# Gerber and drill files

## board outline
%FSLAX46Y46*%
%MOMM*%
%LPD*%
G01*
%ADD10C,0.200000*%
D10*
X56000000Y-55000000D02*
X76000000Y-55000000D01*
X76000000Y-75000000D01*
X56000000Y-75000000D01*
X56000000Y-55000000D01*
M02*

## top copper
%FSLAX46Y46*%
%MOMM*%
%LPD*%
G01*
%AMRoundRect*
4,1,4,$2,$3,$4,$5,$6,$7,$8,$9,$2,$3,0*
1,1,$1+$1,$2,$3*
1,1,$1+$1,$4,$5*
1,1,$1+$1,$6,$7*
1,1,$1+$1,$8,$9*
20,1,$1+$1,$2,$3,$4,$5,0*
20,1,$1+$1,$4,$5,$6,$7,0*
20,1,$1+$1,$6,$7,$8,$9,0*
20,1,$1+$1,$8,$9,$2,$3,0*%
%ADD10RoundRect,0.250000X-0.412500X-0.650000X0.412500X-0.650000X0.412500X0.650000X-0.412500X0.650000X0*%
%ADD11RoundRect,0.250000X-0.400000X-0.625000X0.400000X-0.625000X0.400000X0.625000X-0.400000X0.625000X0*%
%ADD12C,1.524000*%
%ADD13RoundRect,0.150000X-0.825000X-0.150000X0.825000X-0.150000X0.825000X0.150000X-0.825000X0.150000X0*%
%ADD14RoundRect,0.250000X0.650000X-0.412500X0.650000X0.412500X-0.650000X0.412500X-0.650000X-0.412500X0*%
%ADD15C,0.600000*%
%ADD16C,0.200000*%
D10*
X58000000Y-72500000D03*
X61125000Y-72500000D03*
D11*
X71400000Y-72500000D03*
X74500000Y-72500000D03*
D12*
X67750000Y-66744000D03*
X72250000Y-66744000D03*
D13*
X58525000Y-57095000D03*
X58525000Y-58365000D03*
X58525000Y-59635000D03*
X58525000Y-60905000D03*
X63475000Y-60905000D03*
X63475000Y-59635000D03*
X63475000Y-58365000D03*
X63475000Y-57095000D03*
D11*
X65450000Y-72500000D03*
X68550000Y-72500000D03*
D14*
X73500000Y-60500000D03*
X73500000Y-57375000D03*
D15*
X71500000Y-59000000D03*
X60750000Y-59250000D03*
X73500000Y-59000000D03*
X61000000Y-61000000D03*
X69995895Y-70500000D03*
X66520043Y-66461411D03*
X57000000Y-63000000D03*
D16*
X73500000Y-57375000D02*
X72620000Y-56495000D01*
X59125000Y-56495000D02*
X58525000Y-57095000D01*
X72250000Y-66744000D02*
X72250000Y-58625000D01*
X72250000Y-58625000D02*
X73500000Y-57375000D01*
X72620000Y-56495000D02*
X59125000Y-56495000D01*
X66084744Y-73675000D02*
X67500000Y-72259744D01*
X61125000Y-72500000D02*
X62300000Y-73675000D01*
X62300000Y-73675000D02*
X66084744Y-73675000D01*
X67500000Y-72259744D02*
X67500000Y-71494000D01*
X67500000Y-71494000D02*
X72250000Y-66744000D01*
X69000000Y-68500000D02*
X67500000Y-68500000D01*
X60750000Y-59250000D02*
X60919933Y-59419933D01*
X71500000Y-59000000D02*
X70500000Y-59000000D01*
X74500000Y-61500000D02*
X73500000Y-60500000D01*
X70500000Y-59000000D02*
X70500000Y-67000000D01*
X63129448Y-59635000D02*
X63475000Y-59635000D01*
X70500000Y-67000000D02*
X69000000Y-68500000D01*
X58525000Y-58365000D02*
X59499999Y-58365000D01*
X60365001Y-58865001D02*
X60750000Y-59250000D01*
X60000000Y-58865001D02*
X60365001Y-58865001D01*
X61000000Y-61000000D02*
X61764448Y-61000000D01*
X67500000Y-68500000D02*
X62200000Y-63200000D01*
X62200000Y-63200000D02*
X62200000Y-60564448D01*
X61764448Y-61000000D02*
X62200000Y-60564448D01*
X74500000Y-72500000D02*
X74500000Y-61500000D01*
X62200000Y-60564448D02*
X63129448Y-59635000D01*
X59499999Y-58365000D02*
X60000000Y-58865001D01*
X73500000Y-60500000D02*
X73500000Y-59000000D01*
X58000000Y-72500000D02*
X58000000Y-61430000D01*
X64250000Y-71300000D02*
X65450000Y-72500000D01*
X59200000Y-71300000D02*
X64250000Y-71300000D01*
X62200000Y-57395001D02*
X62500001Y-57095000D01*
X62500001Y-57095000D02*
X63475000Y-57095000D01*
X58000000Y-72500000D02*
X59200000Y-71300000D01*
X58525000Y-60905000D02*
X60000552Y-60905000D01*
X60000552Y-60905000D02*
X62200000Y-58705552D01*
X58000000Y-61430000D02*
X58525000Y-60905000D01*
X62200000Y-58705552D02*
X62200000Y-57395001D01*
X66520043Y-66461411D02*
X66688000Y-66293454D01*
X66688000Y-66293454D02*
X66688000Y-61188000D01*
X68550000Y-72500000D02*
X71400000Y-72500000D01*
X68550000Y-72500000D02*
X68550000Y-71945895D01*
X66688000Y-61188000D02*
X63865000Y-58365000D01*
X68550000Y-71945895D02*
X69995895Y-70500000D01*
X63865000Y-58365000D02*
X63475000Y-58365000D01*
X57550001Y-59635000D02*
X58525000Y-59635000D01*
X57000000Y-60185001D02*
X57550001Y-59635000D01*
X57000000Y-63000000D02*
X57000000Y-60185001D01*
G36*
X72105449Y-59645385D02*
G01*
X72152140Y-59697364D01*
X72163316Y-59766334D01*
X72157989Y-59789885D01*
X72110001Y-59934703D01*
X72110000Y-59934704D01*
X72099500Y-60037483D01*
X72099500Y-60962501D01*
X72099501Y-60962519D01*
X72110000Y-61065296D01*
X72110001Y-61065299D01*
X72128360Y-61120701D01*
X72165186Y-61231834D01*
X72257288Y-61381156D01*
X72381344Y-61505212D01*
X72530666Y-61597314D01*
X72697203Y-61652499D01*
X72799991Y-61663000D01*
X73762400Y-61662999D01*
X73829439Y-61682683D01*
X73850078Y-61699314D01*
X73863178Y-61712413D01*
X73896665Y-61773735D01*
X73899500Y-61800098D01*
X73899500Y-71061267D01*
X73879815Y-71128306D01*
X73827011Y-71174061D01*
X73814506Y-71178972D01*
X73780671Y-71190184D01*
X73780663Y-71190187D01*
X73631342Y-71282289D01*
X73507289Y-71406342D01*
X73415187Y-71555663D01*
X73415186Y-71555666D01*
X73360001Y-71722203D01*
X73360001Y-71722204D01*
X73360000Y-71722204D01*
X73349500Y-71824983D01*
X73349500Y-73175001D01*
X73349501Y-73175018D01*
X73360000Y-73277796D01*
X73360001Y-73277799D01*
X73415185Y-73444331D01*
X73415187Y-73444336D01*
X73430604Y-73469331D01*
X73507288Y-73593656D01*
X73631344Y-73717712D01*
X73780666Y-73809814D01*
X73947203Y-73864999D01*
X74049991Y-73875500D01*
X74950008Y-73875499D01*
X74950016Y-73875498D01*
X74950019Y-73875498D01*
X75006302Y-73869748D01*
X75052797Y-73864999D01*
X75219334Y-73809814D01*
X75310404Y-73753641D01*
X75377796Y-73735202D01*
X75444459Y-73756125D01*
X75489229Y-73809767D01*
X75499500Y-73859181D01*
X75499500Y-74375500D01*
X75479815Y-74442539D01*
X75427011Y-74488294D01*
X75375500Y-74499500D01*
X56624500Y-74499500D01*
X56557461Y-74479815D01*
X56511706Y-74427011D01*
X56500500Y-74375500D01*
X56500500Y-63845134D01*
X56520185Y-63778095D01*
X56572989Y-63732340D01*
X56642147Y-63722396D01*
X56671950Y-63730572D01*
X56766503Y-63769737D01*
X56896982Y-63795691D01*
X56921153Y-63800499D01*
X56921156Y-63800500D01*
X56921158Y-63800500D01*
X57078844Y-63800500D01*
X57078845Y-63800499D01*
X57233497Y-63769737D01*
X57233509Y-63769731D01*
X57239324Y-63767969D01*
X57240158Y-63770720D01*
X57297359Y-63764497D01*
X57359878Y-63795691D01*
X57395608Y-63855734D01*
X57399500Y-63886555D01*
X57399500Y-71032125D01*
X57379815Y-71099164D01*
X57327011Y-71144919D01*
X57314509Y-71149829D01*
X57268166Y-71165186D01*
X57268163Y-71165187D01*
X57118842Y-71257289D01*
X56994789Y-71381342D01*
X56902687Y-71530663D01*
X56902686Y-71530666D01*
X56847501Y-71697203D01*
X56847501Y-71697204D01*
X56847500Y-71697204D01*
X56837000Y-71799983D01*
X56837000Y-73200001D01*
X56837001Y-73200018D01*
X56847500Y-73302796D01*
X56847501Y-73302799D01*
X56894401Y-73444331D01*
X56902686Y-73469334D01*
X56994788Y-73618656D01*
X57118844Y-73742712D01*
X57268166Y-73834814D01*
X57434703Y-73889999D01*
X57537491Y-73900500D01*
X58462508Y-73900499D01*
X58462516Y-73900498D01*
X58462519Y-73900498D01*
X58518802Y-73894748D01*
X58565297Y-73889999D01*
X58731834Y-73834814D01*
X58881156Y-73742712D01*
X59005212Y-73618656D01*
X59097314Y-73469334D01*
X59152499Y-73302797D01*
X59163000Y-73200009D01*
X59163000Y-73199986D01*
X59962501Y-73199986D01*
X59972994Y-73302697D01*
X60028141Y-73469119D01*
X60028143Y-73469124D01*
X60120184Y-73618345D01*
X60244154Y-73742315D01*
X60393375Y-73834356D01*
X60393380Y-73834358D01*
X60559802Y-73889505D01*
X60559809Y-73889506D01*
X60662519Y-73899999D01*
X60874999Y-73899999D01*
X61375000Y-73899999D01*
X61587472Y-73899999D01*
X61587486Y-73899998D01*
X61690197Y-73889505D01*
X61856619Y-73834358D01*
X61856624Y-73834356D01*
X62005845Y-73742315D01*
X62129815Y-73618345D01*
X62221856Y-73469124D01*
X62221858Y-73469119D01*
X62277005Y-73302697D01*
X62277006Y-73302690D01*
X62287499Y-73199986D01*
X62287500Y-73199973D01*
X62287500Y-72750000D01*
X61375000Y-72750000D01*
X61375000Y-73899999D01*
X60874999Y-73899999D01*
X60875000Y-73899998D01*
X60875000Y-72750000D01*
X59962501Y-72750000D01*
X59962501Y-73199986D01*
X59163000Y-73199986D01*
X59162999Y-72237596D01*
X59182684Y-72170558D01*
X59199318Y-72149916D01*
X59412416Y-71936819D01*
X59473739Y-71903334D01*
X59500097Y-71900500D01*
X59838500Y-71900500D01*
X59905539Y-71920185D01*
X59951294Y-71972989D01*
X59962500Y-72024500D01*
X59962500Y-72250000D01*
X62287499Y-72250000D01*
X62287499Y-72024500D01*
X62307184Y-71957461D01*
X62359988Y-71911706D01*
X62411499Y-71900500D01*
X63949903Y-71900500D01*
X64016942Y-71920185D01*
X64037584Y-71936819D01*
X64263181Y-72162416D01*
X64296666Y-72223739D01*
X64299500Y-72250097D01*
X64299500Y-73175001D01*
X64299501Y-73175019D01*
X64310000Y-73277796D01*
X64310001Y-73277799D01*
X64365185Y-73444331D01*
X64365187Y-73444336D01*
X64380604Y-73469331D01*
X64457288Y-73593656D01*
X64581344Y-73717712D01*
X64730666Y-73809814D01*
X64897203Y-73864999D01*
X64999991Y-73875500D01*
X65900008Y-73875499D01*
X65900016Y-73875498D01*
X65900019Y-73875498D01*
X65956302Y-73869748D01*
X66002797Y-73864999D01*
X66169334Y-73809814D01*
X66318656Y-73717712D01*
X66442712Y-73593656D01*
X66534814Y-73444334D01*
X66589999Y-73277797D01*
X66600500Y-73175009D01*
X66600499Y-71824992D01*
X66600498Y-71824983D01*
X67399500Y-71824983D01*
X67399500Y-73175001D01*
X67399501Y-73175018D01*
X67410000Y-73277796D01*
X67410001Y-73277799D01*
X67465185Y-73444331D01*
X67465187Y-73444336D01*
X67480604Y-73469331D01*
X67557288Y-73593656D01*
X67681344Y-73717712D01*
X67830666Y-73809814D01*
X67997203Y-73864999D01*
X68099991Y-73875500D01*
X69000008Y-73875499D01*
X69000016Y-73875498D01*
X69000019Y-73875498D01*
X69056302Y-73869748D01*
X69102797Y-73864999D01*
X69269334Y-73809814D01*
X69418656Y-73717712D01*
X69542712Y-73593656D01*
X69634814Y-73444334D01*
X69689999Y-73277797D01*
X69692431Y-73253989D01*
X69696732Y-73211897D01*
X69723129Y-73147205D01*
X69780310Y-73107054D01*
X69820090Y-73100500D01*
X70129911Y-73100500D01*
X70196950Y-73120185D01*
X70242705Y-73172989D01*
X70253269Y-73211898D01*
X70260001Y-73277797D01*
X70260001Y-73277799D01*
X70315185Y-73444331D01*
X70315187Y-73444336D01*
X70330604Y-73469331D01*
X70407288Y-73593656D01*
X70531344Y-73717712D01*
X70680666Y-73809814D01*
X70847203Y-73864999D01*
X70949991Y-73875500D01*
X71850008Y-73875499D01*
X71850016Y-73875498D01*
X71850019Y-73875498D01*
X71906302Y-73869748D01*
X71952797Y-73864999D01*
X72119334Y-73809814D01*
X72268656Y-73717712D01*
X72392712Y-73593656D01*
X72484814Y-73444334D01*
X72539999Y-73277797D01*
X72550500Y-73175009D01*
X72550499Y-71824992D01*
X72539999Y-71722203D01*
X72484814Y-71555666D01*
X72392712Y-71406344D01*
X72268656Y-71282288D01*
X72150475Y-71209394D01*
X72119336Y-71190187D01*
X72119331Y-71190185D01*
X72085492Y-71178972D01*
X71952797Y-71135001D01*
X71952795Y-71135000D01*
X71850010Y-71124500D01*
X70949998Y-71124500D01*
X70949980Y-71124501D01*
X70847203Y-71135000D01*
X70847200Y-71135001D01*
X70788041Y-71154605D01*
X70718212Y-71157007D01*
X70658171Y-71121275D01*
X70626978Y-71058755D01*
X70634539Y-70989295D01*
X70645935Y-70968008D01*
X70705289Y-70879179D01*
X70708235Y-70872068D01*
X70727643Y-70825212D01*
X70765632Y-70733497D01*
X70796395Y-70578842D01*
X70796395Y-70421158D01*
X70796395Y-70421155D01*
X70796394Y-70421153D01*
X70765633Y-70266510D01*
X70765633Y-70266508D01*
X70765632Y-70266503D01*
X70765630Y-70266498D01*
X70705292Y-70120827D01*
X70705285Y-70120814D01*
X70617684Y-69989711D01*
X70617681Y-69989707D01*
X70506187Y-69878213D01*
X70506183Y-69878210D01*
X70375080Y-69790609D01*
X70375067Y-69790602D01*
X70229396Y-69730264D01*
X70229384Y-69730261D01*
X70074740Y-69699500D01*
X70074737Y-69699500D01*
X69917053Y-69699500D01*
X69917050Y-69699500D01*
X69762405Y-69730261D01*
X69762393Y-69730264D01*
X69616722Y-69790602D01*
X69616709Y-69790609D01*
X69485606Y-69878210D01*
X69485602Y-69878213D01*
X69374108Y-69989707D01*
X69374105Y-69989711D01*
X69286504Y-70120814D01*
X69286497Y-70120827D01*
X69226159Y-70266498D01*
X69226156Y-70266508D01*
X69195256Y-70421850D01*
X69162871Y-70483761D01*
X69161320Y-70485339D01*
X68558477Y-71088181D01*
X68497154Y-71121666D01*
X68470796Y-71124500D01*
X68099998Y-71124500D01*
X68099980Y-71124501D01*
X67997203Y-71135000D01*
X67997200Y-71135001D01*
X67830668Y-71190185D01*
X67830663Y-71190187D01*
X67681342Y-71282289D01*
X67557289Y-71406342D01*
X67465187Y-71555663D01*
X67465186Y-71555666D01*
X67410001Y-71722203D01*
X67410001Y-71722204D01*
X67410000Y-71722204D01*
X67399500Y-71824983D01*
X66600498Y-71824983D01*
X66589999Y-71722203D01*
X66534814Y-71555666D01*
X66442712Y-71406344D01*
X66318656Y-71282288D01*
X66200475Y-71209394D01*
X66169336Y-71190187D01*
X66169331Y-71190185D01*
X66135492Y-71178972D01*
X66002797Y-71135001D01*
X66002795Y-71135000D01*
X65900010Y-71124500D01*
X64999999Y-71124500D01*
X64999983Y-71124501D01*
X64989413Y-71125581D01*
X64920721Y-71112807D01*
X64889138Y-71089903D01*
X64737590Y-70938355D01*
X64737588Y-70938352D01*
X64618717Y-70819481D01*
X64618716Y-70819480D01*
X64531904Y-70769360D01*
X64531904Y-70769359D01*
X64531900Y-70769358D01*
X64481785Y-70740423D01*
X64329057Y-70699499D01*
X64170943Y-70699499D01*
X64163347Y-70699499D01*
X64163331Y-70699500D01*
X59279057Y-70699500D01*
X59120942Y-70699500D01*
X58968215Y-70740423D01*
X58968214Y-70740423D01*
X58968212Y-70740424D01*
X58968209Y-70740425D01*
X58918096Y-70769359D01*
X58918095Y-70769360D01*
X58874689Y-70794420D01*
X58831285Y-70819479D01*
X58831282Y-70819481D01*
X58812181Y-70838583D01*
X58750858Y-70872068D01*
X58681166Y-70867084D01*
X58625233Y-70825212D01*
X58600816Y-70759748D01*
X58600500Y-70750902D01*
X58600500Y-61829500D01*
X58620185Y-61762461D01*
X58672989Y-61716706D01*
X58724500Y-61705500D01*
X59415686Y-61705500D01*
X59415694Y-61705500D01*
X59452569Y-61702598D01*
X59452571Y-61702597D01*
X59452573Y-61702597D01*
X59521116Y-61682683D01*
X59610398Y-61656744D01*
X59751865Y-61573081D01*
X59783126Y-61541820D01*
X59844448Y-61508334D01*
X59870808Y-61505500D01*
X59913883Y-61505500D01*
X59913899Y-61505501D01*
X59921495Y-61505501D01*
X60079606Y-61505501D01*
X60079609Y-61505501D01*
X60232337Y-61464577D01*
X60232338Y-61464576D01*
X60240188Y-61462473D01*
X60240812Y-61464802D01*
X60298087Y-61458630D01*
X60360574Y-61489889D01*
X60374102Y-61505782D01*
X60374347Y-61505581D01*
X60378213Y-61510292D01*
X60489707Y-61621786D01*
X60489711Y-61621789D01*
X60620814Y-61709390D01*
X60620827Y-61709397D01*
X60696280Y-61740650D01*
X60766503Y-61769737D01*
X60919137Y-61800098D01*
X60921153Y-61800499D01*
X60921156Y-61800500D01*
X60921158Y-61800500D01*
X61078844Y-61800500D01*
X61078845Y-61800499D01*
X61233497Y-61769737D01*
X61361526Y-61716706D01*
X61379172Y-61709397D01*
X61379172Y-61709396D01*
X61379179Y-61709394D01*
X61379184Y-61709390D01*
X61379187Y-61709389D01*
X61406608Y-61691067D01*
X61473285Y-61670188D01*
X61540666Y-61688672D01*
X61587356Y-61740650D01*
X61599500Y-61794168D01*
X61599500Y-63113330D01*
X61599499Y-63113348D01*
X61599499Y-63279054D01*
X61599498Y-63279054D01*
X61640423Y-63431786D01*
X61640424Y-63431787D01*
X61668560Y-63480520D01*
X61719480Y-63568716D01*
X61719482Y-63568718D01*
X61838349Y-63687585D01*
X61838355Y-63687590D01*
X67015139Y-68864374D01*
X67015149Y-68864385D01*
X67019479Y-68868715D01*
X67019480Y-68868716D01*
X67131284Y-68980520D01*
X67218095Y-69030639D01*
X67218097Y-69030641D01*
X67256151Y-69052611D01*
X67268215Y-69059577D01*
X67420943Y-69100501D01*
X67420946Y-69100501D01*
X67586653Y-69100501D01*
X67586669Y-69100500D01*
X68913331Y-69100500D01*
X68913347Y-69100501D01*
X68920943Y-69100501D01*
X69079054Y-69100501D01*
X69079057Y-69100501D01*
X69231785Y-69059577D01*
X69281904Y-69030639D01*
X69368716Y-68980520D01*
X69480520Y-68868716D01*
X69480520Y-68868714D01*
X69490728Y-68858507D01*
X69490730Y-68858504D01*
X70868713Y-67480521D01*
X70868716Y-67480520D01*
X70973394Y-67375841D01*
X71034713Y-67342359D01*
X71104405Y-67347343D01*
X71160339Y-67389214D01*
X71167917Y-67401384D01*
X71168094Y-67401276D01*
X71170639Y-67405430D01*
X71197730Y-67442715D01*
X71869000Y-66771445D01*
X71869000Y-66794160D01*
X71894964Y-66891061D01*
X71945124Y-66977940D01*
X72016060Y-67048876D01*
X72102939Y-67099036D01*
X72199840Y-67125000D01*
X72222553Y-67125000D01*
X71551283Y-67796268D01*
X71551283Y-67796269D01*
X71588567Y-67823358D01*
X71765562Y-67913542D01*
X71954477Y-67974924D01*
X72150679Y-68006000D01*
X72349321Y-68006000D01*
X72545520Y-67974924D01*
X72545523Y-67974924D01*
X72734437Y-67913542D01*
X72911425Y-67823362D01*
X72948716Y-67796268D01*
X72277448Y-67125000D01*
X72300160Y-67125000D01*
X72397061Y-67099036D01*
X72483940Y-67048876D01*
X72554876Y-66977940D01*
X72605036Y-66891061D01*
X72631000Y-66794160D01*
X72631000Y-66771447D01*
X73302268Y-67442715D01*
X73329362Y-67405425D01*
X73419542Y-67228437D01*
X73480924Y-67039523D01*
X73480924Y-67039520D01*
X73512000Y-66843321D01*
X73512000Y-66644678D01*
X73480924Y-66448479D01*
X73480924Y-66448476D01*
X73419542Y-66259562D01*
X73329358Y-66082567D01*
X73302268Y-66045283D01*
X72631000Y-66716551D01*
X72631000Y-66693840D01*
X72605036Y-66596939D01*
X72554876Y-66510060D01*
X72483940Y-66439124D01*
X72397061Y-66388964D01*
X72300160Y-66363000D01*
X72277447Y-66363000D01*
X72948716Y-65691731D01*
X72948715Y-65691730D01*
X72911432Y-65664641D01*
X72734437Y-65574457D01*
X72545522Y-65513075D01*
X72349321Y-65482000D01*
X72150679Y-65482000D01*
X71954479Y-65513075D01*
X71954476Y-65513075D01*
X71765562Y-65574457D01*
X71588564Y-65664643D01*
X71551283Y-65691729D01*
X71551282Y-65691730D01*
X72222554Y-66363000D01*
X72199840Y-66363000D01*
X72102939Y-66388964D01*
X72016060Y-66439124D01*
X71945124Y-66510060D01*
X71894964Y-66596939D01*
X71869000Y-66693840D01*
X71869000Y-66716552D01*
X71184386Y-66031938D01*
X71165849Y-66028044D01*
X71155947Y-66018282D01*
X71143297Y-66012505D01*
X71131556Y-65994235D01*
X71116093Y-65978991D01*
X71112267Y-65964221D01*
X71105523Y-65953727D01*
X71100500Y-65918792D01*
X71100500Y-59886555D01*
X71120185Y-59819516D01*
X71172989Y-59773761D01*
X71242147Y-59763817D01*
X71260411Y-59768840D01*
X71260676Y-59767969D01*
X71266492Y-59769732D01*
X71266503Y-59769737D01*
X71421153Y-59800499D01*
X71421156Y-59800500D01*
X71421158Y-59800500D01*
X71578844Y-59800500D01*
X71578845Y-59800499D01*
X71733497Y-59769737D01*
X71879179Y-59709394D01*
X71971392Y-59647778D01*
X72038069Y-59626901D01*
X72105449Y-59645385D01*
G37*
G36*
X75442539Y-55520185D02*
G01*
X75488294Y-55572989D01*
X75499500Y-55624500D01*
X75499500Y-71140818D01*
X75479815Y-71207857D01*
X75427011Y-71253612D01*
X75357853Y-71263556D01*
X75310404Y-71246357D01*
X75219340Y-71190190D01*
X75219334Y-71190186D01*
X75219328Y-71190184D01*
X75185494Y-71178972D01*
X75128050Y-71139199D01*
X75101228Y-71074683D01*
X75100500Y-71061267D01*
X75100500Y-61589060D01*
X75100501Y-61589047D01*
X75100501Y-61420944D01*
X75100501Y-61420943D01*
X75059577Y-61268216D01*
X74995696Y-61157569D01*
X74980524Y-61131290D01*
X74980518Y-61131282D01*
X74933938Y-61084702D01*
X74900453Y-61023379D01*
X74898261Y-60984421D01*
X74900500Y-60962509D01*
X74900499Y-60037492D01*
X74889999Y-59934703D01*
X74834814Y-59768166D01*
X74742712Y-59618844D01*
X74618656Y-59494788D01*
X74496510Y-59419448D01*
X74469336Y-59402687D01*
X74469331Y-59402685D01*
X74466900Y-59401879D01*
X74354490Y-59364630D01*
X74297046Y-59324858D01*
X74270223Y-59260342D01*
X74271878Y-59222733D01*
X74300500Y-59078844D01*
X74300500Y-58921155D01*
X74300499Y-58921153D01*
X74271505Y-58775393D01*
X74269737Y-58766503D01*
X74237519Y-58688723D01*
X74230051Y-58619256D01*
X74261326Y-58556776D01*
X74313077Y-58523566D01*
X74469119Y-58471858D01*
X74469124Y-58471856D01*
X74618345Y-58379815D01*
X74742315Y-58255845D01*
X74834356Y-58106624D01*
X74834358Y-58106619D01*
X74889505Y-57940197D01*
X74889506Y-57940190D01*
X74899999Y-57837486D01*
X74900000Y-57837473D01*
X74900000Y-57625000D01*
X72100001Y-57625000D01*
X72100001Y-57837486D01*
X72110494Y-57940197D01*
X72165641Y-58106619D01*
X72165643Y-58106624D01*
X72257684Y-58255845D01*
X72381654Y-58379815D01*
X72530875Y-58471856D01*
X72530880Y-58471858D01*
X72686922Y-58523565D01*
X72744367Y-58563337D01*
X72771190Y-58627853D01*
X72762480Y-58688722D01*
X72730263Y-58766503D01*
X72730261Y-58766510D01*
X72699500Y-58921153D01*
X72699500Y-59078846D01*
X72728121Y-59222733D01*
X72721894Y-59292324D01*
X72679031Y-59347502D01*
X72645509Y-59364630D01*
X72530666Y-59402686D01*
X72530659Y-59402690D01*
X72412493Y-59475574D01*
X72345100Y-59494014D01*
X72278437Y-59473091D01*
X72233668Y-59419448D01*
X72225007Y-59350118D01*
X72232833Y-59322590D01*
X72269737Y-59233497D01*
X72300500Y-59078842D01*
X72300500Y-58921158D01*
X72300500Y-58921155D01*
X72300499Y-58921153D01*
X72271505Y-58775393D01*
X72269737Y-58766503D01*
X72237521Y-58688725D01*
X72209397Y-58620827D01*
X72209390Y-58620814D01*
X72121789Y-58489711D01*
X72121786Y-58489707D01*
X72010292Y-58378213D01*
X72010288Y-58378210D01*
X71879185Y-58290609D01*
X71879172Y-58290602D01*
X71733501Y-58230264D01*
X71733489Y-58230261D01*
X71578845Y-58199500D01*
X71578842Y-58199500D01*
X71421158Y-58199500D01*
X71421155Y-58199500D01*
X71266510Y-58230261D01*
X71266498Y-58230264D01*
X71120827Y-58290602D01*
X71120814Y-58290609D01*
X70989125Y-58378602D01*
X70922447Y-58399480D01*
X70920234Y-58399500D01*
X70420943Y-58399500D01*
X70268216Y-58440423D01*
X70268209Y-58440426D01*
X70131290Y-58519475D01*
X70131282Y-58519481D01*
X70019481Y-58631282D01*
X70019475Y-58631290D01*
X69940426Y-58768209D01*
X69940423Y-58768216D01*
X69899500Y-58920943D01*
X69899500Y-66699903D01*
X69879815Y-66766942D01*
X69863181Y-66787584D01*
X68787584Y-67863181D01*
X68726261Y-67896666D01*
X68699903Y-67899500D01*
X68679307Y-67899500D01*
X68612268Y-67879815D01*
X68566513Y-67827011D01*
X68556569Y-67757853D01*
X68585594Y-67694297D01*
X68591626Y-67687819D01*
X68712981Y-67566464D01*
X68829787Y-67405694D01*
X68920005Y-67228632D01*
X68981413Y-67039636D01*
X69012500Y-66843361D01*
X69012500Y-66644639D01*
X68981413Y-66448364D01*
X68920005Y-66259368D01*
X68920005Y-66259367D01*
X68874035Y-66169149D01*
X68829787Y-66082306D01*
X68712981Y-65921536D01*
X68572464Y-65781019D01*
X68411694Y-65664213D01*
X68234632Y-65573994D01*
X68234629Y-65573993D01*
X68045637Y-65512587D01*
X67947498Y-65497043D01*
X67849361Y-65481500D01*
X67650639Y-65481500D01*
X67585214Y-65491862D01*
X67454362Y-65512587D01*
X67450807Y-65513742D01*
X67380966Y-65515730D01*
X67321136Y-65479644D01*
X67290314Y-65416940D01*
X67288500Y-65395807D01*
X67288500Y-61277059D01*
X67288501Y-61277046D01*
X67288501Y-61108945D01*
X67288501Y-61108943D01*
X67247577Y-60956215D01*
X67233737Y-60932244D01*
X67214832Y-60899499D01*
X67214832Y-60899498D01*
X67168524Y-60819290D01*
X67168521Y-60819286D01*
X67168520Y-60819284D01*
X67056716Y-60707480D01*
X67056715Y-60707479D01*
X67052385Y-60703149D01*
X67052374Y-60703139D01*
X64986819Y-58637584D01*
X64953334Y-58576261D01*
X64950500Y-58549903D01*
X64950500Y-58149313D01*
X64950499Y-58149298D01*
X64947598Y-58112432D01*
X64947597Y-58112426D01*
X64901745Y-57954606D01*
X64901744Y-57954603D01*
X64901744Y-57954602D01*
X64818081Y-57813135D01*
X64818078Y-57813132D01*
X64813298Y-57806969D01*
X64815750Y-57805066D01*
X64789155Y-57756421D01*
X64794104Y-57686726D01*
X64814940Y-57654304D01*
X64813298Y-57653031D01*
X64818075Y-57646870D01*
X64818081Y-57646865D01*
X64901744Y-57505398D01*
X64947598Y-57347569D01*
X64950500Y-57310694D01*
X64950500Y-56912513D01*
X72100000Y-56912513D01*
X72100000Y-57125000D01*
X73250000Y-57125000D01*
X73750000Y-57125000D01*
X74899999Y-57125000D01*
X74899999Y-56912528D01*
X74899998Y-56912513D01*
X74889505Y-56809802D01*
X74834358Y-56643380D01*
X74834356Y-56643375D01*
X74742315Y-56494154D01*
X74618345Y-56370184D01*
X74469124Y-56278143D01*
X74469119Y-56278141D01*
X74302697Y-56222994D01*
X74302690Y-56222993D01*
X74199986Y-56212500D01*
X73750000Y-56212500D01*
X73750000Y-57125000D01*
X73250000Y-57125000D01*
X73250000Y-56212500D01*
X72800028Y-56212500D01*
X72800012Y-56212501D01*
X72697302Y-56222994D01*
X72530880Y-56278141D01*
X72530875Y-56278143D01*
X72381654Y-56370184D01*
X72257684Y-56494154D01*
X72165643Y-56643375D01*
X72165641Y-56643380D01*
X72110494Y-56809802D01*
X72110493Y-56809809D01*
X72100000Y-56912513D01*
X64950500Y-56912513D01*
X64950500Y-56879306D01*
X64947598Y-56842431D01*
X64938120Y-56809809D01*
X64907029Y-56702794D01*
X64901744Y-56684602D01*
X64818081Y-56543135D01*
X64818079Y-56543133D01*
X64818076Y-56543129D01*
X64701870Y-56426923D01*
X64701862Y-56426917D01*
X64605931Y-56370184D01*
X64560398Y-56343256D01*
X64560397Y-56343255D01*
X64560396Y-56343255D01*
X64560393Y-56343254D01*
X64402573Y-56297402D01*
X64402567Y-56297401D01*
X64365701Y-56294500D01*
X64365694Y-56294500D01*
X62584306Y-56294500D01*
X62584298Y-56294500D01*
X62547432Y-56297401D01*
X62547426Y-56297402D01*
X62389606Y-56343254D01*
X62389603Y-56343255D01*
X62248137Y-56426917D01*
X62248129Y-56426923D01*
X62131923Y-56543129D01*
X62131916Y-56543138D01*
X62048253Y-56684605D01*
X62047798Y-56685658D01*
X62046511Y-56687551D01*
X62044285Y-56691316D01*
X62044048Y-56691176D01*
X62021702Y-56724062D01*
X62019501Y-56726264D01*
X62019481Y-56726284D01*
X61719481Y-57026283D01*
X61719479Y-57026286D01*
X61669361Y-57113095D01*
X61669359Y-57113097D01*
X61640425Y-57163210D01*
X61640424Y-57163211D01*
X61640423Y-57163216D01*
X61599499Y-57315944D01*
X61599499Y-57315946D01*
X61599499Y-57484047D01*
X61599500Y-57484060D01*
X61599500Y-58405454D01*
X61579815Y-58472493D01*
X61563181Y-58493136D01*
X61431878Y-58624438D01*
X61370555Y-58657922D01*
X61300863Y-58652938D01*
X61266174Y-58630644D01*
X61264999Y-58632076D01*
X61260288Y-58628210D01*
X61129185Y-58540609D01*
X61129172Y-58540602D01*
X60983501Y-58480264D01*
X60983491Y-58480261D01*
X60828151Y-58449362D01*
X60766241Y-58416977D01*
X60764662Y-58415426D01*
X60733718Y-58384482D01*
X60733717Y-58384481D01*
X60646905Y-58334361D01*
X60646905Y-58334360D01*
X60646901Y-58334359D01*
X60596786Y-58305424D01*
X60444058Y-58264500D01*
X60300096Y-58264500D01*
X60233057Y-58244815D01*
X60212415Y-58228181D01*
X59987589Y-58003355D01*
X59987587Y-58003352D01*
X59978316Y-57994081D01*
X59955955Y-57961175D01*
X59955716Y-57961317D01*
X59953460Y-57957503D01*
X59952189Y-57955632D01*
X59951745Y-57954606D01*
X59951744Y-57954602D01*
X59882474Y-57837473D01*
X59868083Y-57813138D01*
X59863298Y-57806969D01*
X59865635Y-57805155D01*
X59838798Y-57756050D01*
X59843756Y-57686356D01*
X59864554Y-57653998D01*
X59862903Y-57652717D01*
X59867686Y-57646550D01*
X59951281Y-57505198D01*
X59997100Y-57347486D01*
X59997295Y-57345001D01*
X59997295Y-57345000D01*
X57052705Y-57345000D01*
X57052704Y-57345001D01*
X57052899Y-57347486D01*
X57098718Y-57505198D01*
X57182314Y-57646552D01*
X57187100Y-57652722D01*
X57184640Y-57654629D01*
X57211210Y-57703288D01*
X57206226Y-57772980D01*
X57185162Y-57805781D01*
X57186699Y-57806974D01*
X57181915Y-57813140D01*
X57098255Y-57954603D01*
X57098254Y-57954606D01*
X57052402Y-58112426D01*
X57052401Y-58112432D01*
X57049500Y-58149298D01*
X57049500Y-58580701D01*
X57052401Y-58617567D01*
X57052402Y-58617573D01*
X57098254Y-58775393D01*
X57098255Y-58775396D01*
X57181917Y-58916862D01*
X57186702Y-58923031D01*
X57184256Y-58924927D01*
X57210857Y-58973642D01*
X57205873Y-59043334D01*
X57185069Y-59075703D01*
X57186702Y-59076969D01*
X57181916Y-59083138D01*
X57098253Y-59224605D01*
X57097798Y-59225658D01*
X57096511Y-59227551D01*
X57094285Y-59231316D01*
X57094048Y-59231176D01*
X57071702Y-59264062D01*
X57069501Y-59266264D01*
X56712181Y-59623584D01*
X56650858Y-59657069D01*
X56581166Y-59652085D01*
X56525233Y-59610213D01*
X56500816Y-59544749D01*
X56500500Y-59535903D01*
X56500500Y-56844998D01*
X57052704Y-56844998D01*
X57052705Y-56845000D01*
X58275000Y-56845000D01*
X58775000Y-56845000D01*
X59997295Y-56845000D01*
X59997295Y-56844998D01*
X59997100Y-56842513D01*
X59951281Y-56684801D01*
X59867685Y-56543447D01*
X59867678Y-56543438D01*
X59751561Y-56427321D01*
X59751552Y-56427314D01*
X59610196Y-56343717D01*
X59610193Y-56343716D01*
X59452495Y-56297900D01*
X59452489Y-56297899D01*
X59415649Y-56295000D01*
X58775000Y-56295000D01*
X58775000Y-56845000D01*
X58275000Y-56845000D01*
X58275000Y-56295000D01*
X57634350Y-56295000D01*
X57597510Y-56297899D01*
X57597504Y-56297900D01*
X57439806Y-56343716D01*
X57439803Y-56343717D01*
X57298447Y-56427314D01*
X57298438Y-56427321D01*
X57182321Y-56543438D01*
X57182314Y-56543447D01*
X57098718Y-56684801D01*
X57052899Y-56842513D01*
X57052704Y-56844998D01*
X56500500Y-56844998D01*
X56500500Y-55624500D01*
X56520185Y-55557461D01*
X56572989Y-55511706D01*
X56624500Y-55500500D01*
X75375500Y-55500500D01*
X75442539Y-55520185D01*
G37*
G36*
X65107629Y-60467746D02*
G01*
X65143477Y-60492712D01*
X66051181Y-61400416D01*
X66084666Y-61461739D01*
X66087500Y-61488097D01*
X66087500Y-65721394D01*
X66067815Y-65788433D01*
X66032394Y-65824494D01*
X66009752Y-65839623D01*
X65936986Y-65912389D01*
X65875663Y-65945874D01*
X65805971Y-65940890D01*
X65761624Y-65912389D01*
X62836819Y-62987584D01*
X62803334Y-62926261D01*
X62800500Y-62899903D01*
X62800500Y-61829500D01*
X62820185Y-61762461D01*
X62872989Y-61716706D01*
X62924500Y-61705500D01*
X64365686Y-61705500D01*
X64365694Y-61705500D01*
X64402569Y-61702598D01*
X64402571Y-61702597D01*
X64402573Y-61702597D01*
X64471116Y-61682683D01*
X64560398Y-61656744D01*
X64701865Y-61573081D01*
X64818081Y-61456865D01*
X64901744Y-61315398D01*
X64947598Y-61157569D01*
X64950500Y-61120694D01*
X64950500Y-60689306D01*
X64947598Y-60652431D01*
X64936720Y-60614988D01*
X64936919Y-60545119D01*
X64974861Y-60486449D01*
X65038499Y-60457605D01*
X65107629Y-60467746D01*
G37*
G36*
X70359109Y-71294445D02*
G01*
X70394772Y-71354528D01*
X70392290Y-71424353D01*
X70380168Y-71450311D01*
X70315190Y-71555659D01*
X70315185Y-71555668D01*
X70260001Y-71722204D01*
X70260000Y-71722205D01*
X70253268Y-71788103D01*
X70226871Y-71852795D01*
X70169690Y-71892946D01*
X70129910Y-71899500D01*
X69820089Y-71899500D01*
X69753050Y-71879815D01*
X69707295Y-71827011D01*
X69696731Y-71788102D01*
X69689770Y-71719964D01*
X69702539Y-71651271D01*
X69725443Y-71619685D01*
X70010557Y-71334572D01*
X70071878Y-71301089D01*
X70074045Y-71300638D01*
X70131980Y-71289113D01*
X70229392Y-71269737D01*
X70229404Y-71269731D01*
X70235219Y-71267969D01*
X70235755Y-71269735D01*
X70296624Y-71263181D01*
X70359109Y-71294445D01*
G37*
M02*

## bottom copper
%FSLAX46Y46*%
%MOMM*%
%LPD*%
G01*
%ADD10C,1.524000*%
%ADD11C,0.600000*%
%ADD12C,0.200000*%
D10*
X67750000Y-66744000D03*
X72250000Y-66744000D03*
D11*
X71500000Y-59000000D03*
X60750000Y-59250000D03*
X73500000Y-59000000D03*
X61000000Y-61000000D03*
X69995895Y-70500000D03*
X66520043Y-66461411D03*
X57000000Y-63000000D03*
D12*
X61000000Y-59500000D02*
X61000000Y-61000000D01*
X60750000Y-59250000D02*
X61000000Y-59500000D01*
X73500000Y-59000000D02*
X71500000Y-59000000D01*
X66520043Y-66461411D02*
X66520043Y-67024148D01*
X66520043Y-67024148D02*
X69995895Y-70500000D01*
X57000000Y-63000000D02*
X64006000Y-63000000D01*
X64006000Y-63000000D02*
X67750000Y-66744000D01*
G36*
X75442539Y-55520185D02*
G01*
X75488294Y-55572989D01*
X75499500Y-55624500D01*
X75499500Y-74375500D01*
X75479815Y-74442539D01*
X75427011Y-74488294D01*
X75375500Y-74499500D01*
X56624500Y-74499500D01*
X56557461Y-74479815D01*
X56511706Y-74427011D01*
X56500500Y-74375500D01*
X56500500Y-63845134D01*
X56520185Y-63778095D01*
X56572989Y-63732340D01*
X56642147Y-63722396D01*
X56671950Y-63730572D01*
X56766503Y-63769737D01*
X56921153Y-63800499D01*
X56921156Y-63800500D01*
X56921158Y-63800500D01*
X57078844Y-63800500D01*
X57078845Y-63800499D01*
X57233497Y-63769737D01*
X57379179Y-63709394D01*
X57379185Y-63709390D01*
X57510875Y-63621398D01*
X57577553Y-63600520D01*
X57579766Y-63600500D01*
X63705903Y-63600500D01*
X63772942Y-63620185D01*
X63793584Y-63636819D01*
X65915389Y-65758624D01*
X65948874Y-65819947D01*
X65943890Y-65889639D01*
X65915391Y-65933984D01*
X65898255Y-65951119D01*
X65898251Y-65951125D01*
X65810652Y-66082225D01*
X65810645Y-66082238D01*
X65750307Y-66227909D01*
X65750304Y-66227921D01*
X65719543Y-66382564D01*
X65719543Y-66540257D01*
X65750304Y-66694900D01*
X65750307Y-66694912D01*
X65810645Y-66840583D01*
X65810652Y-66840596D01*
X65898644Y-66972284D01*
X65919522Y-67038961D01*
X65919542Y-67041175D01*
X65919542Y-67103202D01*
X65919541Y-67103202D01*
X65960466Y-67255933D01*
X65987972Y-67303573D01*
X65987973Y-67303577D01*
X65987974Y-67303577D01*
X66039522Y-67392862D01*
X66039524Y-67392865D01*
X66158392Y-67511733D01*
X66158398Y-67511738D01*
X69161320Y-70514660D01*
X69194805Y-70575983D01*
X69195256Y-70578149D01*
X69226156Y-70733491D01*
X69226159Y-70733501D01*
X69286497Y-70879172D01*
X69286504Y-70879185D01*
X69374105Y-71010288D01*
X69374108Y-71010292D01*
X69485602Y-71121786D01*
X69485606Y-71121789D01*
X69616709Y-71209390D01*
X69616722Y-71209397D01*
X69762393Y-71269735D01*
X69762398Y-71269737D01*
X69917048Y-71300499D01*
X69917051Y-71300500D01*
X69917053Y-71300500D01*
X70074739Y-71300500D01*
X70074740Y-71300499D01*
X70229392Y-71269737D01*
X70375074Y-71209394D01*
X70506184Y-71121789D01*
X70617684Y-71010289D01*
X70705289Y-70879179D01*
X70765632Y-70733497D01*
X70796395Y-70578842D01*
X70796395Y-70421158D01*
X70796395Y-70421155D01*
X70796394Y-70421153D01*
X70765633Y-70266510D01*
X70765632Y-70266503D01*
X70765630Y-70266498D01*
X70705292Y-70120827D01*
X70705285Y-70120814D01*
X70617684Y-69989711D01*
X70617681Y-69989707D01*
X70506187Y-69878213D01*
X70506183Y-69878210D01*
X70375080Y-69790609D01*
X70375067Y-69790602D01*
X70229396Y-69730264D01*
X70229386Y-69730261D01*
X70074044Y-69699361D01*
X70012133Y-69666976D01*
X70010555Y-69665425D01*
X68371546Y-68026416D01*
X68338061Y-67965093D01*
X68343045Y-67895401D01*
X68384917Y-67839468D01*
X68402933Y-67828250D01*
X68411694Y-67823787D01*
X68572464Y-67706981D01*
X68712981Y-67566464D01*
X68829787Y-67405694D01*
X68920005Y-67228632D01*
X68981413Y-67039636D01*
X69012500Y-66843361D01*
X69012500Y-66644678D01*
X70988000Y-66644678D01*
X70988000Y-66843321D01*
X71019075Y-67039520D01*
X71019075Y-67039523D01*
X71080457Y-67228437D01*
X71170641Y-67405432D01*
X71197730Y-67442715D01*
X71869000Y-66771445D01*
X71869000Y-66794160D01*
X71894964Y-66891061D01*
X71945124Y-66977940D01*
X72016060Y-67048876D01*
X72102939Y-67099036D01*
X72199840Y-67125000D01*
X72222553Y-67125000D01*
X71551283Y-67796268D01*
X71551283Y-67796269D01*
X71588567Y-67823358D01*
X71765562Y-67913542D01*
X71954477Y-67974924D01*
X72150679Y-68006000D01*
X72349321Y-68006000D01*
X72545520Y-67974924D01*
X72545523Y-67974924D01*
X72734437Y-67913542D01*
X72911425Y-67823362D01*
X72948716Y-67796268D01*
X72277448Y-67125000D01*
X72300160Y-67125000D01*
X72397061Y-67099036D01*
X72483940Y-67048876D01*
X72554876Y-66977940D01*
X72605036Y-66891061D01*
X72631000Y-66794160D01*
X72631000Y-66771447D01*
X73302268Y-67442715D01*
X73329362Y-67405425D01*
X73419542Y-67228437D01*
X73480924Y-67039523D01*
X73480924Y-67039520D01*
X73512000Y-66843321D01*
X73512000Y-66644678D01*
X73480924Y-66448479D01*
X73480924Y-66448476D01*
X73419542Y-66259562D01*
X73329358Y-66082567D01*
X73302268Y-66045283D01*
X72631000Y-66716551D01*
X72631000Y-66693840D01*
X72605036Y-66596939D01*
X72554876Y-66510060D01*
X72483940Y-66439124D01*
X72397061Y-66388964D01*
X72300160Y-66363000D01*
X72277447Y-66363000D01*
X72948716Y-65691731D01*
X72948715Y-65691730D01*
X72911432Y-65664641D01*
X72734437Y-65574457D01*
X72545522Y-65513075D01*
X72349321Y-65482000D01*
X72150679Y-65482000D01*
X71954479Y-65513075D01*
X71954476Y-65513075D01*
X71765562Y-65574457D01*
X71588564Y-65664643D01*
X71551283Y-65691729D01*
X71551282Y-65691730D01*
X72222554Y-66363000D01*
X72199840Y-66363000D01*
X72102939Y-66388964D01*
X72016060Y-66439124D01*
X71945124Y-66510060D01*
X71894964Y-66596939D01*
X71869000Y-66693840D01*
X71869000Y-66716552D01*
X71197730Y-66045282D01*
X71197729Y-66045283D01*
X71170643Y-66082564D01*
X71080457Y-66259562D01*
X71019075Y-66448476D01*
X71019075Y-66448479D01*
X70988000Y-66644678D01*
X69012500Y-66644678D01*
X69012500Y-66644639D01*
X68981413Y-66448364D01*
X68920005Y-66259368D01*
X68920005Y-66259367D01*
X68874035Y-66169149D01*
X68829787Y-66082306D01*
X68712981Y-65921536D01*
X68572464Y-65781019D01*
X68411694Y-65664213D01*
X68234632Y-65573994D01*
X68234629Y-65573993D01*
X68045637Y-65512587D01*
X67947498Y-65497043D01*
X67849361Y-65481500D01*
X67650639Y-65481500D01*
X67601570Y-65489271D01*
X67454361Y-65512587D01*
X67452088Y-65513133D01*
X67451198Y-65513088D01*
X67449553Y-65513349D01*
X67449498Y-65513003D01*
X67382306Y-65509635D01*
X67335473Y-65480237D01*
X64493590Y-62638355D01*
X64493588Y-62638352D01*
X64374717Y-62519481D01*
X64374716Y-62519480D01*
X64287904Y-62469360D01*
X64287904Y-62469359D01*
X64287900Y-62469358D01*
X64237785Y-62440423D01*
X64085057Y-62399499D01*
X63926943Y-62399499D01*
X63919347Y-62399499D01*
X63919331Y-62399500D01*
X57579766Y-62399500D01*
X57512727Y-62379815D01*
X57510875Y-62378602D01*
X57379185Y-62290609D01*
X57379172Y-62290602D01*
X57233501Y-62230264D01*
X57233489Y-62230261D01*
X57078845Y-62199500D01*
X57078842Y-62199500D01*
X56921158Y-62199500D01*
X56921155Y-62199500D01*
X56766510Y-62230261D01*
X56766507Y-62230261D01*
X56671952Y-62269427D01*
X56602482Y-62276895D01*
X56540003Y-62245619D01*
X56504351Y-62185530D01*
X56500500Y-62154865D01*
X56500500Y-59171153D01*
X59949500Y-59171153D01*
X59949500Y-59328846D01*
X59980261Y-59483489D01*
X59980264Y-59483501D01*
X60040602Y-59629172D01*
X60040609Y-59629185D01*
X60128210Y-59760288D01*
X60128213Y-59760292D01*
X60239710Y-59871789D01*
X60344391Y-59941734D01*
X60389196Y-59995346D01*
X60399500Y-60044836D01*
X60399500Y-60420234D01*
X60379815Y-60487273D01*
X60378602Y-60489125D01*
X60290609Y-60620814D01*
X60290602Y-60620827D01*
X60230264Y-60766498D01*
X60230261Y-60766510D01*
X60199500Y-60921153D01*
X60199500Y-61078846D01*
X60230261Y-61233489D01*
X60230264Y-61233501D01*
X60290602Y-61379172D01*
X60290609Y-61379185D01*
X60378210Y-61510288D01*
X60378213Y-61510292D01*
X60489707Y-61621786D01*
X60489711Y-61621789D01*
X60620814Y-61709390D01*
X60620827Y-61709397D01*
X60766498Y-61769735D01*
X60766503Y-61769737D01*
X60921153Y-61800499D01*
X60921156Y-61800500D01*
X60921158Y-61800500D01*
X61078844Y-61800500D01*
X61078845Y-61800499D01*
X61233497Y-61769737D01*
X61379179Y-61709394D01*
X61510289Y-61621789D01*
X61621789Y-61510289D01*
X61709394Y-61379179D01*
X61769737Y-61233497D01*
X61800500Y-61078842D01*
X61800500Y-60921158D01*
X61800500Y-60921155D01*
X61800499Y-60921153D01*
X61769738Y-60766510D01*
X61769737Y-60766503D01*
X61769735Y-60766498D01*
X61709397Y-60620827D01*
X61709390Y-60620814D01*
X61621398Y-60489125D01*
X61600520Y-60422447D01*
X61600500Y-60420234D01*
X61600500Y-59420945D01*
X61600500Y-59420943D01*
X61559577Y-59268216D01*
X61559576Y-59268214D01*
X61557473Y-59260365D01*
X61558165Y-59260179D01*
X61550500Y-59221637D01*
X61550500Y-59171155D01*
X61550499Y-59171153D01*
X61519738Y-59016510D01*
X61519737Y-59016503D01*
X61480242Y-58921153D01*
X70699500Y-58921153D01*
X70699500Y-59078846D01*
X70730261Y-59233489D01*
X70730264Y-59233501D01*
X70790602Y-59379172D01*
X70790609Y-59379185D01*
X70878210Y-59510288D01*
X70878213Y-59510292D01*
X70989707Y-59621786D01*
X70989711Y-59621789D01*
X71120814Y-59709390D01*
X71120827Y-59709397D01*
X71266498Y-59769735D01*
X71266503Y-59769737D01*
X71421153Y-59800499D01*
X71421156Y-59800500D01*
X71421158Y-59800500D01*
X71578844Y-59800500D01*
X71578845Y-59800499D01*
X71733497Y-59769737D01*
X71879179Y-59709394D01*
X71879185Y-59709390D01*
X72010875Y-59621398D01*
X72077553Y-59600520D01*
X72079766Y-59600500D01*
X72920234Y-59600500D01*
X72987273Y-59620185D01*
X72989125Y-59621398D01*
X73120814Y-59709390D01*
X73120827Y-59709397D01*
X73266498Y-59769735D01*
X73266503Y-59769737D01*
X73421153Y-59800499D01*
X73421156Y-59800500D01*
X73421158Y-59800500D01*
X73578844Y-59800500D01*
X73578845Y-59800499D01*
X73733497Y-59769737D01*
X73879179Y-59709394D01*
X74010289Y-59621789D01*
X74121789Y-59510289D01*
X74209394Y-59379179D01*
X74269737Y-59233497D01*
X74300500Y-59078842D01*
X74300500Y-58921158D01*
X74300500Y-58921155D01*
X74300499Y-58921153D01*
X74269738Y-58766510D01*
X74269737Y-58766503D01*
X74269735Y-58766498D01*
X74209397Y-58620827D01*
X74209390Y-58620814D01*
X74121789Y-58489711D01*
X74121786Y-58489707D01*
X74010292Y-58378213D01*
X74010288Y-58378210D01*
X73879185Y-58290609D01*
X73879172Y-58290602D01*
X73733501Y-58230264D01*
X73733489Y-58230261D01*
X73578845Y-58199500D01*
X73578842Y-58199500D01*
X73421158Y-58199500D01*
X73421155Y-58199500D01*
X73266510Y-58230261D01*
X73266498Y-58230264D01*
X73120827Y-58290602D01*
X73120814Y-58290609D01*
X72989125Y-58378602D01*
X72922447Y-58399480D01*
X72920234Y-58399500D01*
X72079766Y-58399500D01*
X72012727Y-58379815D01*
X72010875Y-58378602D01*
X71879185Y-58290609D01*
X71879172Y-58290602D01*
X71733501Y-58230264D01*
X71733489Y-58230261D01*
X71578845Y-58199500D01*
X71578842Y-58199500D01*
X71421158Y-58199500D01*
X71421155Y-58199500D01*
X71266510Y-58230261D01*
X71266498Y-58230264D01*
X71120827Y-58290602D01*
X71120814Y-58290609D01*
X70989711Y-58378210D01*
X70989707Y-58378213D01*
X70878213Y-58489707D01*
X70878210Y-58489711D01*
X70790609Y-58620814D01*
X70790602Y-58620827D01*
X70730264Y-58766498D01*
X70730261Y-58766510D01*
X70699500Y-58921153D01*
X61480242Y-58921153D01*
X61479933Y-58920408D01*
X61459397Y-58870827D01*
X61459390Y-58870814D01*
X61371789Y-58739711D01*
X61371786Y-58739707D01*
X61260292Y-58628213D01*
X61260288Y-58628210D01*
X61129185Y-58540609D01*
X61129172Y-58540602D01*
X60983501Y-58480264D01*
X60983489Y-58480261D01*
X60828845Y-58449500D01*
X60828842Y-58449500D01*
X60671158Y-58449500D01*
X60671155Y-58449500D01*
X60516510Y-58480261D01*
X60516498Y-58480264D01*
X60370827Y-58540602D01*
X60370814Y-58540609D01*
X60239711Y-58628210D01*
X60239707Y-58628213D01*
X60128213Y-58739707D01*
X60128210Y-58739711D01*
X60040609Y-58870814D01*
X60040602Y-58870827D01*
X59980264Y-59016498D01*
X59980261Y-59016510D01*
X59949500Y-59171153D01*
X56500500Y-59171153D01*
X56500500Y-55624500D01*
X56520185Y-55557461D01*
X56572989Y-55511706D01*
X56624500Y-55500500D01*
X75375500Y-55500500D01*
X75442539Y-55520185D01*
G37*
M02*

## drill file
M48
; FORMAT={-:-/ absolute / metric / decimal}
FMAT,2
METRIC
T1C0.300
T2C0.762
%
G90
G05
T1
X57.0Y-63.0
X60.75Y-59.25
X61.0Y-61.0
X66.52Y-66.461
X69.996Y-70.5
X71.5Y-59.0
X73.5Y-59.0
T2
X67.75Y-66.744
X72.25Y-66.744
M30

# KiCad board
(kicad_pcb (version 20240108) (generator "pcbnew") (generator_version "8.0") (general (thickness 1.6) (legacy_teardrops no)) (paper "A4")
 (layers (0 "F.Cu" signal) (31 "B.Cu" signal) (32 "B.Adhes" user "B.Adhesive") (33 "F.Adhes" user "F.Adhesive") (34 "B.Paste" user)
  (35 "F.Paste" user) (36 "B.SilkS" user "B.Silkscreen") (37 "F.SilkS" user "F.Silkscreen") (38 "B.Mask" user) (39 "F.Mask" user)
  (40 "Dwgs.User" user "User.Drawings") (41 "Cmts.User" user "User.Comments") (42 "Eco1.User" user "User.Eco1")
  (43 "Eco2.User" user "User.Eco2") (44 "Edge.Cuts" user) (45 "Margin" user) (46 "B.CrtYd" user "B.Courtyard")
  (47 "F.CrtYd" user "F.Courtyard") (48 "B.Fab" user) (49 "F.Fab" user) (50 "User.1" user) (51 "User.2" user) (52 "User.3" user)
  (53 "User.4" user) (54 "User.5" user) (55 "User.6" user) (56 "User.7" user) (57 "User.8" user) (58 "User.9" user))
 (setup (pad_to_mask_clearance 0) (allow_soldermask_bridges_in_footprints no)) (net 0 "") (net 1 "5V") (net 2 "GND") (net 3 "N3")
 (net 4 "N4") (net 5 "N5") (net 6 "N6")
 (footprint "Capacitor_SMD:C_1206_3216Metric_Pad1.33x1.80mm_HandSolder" (layer "F.Cu") (at 59.5625 72.5)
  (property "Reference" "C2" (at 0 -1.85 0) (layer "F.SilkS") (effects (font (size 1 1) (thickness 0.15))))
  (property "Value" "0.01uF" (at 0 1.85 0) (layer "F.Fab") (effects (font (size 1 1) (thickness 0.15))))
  (pad "1" smd roundrect (at -1.5625 0) (size 1.325 1.8) (layers "F.Cu" "F.Paste" "F.Mask") (roundrect_rratio 0.188679) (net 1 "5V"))
  (pad "2" smd roundrect (at 1.5625 0) (size 1.325 1.8) (layers "F.Cu" "F.Paste" "F.Mask") (roundrect_rratio 0.188679) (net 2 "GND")))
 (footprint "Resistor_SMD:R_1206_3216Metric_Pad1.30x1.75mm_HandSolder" (layer "F.Cu") (at 72.95 72.5)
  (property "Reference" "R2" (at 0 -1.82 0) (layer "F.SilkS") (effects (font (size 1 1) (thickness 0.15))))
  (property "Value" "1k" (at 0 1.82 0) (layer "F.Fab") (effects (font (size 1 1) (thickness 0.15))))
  (pad "1" smd roundrect (at -1.55 0) (size 1.3 1.75) (layers "F.Cu" "F.Paste" "F.Mask") (roundrect_rratio 0.192308) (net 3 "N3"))
  (pad "2" smd roundrect (at 1.55 0) (size 1.3 1.75) (layers "F.Cu" "F.Paste" "F.Mask") (roundrect_rratio 0.192308) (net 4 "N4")))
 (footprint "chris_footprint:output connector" (layer "F.Cu") (at 69.75 64.744)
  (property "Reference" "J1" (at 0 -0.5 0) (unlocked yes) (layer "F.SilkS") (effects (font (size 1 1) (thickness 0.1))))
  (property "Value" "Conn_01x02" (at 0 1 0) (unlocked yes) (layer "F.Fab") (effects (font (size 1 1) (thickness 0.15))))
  (pad "1" thru_hole circle (at -2 2) (size 1.524 1.524) (drill 0.762) (layers "*.Cu" "*.Mask") (remove_unused_layers no) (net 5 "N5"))
  (pad "2" thru_hole circle (at 2.5 2) (size 1.524 1.524) (drill 0.762) (layers "*.Cu" "*.Mask") (remove_unused_layers no) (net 2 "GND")))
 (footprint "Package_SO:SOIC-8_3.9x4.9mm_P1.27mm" (layer "F.Cu") (at 61 59)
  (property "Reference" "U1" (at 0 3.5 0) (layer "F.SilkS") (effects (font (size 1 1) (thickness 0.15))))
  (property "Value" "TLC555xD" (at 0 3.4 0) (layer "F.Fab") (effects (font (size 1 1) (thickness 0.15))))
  (pad "1" smd roundrect (at -2.475 -1.905) (size 1.95 0.6) (layers "F.Cu" "F.Paste" "F.Mask") (roundrect_rratio 0.25) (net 2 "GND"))
  (pad "2" smd roundrect (at -2.475 -0.635) (size 1.95 0.6) (layers "F.Cu" "F.Paste" "F.Mask") (roundrect_rratio 0.25) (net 4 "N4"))
  (pad "3" smd roundrect (at -2.475 0.635) (size 1.95 0.6) (layers "F.Cu" "F.Paste" "F.Mask") (roundrect_rratio 0.25) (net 5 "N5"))
  (pad "4" smd roundrect (at -2.475 1.905) (size 1.95 0.6) (layers "F.Cu" "F.Paste" "F.Mask") (roundrect_rratio 0.25) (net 1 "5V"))
  (pad "5" smd roundrect (at 2.475 1.905) (size 1.95 0.6) (layers "F.Cu" "F.Paste" "F.Mask") (roundrect_rratio 0.25) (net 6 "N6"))
  (pad "6" smd roundrect (at 2.475 0.635) (size 1.95 0.6) (layers "F.Cu" "F.Paste" "F.Mask") (roundrect_rratio 0.25) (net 4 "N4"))
  (pad "7" smd roundrect (at 2.475 -0.635) (size 1.95 0.6) (layers "F.Cu" "F.Paste" "F.Mask") (roundrect_rratio 0.25) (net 3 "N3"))
  (pad "8" smd roundrect (at 2.475 -1.905) (size 1.95 0.6) (layers "F.Cu" "F.Paste" "F.Mask") (roundrect_rratio 0.25) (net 1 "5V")))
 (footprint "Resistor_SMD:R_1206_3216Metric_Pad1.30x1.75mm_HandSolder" (layer "F.Cu") (at 67 72.5)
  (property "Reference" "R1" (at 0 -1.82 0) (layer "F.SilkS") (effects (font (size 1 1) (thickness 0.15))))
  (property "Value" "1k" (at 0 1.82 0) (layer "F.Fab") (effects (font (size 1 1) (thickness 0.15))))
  (pad "1" smd roundrect (at -1.55 0) (size 1.3 1.75) (layers "F.Cu" "F.Paste" "F.Mask") (roundrect_rratio 0.192308) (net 1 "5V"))
  (pad "2" smd roundrect (at 1.55 0) (size 1.3 1.75) (layers "F.Cu" "F.Paste" "F.Mask") (roundrect_rratio 0.192308) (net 3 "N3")))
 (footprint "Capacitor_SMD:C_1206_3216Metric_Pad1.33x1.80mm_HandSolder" (layer "F.Cu") (at 73.5 58.9375 90)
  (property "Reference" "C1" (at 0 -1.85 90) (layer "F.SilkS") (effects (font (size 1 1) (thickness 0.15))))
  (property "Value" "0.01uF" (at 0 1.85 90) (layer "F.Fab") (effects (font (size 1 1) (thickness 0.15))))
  (pad "1" smd roundrect (at -1.5625 0 90) (size 1.325 1.8) (layers "F.Cu" "F.Paste" "F.Mask") (roundrect_rratio 0.188679) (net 4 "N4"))
  (pad "2" smd roundrect (at 1.5625 0 90) (size 1.325 1.8) (layers "F.Cu" "F.Paste" "F.Mask") (roundrect_rratio 0.188679) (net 2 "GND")))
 (gr_rect (start 56 55) (end 76 75) (stroke (width 0.2) (type default)) (fill none) (layer "Edge.Cuts"))
 (segment (start 73.5 57.375) (end 72.62 56.495) (width 0.2) (layer "F.Cu") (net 2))
 (segment (start 59.125 56.495) (end 58.525 57.095) (width 0.2) (layer "F.Cu") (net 2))
 (segment (start 72.25 66.744) (end 72.25 58.625) (width 0.2) (layer "F.Cu") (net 2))
 (segment (start 72.25 58.625) (end 73.5 57.375) (width 0.2) (layer "F.Cu") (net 2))
 (segment (start 72.62 56.495) (end 59.125 56.495) (width 0.2) (layer "F.Cu") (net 2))
 (segment (start 66.084744 73.675) (end 67.5 72.259744) (width 0.2) (layer "F.Cu") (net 2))
 (segment (start 61.125 72.5) (end 62.3 73.675) (width 0.2) (layer "F.Cu") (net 2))
 (segment (start 62.3 73.675) (end 66.084744 73.675) (width 0.2) (layer "F.Cu") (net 2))
 (segment (start 67.5 72.259744) (end 67.5 71.494) (width 0.2) (layer "F.Cu") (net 2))
 (segment (start 67.5 71.494) (end 72.25 66.744) (width 0.2) (layer "F.Cu") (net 2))
 (segment (start 69 68.5) (end 67.5 68.5) (width 0.2) (layer "F.Cu") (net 4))
 (segment (start 60.75 59.25) (end 60.919933 59.419933) (width 0.2) (layer "F.Cu") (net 4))
 (segment (start 71.5 59) (end 70.5 59) (width 0.2) (layer "F.Cu") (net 4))
 (segment (start 74.5 61.5) (end 73.5 60.5) (width 0.2) (layer "F.Cu") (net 4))
 (segment (start 70.5 59) (end 70.5 67) (width 0.2) (layer "F.Cu") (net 4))
 (segment (start 63.129448 59.635) (end 63.475 59.635) (width 0.2) (layer "F.Cu") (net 4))
 (segment (start 70.5 67) (end 69 68.5) (width 0.2) (layer "F.Cu") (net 4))
 (segment (start 58.525 58.365) (end 59.499999 58.365) (width 0.2) (layer "F.Cu") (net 4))
 (segment (start 60.365001 58.865001) (end 60.75 59.25) (width 0.2) (layer "F.Cu") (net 4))
 (segment (start 60 58.865001) (end 60.365001 58.865001) (width 0.2) (layer "F.Cu") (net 4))
 (segment (start 61 61) (end 61.764448 61) (width 0.2) (layer "F.Cu") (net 4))
 (segment (start 67.5 68.5) (end 62.2 63.2) (width 0.2) (layer "F.Cu") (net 4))
 (segment (start 62.2 63.2) (end 62.2 60.564448) (width 0.2) (layer "F.Cu") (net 4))
 (segment (start 61.764448 61) (end 62.2 60.564448) (width 0.2) (layer "F.Cu") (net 4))
 (segment (start 74.5 72.5) (end 74.5 61.5) (width 0.2) (layer "F.Cu") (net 4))
 (segment (start 62.2 60.564448) (end 63.129448 59.635) (width 0.2) (layer "F.Cu") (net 4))
 (segment (start 59.499999 58.365) (end 60 58.865001) (width 0.2) (layer "F.Cu") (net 4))
 (segment (start 73.5 60.5) (end 73.5 59) (width 0.2) (layer "F.Cu") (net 4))
 (via (at 71.5 59) (size 0.6) (drill 0.3) (layers "F.Cu" "B.Cu") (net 4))
 (via (at 60.75 59.25) (size 0.6) (drill 0.3) (layers "F.Cu" "B.Cu") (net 4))
 (via (at 73.5 59) (size 0.6) (drill 0.3) (layers "F.Cu" "B.Cu") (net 4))
 (via (at 61 61) (size 0.6) (drill 0.3) (layers "F.Cu" "B.Cu") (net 4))
 (segment (start 61 59.5) (end 61 61) (width 0.2) (layer "B.Cu") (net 4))
 (segment (start 60.75 59.25) (end 61 59.5) (width 0.2) (layer "B.Cu") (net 4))
 (segment (start 73.5 59) (end 71.5 59) (width 0.2) (layer "B.Cu") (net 4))
 (segment (start 58 72.5) (end 58 61.43) (width 0.2) (layer "F.Cu") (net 1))
 (segment (start 64.25 71.3) (end 65.45 72.5) (width 0.2) (layer "F.Cu") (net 1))
 (segment (start 59.2 71.3) (end 64.25 71.3) (width 0.2) (layer "F.Cu") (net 1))
 (segment (start 62.2 57.395001) (end 62.500001 57.095) (width 0.2) (layer "F.Cu") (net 1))
 (segment (start 62.500001 57.095) (end 63.475 57.095) (width 0.2) (layer "F.Cu") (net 1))
 (segment (start 58 72.5) (end 59.2 71.3) (width 0.2) (layer "F.Cu") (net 1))
 (segment (start 58.525 60.905) (end 60.000552 60.905) (width 0.2) (layer "F.Cu") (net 1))
 (segment (start 60.000552 60.905) (end 62.2 58.705552) (width 0.2) (layer "F.Cu") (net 1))
 (segment (start 58 61.43) (end 58.525 60.905) (width 0.2) (layer "F.Cu") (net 1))
 (segment (start 62.2 58.705552) (end 62.2 57.395001) (width 0.2) (layer "F.Cu") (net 1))
 (segment (start 66.520043 66.461411) (end 66.688 66.293454) (width 0.2) (layer "F.Cu") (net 3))
 (segment (start 66.688 66.293454) (end 66.688 61.188) (width 0.2) (layer "F.Cu") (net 3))
 (segment (start 68.55 72.5) (end 71.4 72.5) (width 0.2) (layer "F.Cu") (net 3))
 (segment (start 68.55 72.5) (end 68.55 71.945895) (width 0.2) (layer "F.Cu") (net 3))
 (segment (start 66.688 61.188) (end 63.865 58.365) (width 0.2) (layer "F.Cu") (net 3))
 (segment (start 68.55 71.945895) (end 69.995895 70.5) (width 0.2) (layer "F.Cu") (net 3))
 (segment (start 63.865 58.365) (end 63.475 58.365) (width 0.2) (layer "F.Cu") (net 3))
 (via (at 69.995895 70.5) (size 0.6) (drill 0.3) (layers "F.Cu" "B.Cu") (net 3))
 (via (at 66.520043 66.461411) (size 0.6) (drill 0.3) (layers "F.Cu" "B.Cu") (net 3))
 (segment (start 66.520043 66.461411) (end 66.520043 67.024148) (width 0.2) (layer "B.Cu") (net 3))
 (segment (start 66.520043 67.024148) (end 69.995895 70.5) (width 0.2) (layer "B.Cu") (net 3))
 (segment (start 57.550001 59.635) (end 58.525 59.635) (width 0.2) (layer "F.Cu") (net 5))
 (segment (start 57 60.185001) (end 57.550001 59.635) (width 0.2) (layer "F.Cu") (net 5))
 (segment (start 57 63) (end 57 60.185001) (width 0.2) (layer "F.Cu") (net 5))
 (via (at 57 63) (size 0.6) (drill 0.3) (layers "F.Cu" "B.Cu") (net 5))
 (segment (start 57 63) (end 64.006 63) (width 0.2) (layer "B.Cu") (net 5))
 (segment (start 64.006 63) (end 67.75 66.744) (width 0.2) (layer "B.Cu") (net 5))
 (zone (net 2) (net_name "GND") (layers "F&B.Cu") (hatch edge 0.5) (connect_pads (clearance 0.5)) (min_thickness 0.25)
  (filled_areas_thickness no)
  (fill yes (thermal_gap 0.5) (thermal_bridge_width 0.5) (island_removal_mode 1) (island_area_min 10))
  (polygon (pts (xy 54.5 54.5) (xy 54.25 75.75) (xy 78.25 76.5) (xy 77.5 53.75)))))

